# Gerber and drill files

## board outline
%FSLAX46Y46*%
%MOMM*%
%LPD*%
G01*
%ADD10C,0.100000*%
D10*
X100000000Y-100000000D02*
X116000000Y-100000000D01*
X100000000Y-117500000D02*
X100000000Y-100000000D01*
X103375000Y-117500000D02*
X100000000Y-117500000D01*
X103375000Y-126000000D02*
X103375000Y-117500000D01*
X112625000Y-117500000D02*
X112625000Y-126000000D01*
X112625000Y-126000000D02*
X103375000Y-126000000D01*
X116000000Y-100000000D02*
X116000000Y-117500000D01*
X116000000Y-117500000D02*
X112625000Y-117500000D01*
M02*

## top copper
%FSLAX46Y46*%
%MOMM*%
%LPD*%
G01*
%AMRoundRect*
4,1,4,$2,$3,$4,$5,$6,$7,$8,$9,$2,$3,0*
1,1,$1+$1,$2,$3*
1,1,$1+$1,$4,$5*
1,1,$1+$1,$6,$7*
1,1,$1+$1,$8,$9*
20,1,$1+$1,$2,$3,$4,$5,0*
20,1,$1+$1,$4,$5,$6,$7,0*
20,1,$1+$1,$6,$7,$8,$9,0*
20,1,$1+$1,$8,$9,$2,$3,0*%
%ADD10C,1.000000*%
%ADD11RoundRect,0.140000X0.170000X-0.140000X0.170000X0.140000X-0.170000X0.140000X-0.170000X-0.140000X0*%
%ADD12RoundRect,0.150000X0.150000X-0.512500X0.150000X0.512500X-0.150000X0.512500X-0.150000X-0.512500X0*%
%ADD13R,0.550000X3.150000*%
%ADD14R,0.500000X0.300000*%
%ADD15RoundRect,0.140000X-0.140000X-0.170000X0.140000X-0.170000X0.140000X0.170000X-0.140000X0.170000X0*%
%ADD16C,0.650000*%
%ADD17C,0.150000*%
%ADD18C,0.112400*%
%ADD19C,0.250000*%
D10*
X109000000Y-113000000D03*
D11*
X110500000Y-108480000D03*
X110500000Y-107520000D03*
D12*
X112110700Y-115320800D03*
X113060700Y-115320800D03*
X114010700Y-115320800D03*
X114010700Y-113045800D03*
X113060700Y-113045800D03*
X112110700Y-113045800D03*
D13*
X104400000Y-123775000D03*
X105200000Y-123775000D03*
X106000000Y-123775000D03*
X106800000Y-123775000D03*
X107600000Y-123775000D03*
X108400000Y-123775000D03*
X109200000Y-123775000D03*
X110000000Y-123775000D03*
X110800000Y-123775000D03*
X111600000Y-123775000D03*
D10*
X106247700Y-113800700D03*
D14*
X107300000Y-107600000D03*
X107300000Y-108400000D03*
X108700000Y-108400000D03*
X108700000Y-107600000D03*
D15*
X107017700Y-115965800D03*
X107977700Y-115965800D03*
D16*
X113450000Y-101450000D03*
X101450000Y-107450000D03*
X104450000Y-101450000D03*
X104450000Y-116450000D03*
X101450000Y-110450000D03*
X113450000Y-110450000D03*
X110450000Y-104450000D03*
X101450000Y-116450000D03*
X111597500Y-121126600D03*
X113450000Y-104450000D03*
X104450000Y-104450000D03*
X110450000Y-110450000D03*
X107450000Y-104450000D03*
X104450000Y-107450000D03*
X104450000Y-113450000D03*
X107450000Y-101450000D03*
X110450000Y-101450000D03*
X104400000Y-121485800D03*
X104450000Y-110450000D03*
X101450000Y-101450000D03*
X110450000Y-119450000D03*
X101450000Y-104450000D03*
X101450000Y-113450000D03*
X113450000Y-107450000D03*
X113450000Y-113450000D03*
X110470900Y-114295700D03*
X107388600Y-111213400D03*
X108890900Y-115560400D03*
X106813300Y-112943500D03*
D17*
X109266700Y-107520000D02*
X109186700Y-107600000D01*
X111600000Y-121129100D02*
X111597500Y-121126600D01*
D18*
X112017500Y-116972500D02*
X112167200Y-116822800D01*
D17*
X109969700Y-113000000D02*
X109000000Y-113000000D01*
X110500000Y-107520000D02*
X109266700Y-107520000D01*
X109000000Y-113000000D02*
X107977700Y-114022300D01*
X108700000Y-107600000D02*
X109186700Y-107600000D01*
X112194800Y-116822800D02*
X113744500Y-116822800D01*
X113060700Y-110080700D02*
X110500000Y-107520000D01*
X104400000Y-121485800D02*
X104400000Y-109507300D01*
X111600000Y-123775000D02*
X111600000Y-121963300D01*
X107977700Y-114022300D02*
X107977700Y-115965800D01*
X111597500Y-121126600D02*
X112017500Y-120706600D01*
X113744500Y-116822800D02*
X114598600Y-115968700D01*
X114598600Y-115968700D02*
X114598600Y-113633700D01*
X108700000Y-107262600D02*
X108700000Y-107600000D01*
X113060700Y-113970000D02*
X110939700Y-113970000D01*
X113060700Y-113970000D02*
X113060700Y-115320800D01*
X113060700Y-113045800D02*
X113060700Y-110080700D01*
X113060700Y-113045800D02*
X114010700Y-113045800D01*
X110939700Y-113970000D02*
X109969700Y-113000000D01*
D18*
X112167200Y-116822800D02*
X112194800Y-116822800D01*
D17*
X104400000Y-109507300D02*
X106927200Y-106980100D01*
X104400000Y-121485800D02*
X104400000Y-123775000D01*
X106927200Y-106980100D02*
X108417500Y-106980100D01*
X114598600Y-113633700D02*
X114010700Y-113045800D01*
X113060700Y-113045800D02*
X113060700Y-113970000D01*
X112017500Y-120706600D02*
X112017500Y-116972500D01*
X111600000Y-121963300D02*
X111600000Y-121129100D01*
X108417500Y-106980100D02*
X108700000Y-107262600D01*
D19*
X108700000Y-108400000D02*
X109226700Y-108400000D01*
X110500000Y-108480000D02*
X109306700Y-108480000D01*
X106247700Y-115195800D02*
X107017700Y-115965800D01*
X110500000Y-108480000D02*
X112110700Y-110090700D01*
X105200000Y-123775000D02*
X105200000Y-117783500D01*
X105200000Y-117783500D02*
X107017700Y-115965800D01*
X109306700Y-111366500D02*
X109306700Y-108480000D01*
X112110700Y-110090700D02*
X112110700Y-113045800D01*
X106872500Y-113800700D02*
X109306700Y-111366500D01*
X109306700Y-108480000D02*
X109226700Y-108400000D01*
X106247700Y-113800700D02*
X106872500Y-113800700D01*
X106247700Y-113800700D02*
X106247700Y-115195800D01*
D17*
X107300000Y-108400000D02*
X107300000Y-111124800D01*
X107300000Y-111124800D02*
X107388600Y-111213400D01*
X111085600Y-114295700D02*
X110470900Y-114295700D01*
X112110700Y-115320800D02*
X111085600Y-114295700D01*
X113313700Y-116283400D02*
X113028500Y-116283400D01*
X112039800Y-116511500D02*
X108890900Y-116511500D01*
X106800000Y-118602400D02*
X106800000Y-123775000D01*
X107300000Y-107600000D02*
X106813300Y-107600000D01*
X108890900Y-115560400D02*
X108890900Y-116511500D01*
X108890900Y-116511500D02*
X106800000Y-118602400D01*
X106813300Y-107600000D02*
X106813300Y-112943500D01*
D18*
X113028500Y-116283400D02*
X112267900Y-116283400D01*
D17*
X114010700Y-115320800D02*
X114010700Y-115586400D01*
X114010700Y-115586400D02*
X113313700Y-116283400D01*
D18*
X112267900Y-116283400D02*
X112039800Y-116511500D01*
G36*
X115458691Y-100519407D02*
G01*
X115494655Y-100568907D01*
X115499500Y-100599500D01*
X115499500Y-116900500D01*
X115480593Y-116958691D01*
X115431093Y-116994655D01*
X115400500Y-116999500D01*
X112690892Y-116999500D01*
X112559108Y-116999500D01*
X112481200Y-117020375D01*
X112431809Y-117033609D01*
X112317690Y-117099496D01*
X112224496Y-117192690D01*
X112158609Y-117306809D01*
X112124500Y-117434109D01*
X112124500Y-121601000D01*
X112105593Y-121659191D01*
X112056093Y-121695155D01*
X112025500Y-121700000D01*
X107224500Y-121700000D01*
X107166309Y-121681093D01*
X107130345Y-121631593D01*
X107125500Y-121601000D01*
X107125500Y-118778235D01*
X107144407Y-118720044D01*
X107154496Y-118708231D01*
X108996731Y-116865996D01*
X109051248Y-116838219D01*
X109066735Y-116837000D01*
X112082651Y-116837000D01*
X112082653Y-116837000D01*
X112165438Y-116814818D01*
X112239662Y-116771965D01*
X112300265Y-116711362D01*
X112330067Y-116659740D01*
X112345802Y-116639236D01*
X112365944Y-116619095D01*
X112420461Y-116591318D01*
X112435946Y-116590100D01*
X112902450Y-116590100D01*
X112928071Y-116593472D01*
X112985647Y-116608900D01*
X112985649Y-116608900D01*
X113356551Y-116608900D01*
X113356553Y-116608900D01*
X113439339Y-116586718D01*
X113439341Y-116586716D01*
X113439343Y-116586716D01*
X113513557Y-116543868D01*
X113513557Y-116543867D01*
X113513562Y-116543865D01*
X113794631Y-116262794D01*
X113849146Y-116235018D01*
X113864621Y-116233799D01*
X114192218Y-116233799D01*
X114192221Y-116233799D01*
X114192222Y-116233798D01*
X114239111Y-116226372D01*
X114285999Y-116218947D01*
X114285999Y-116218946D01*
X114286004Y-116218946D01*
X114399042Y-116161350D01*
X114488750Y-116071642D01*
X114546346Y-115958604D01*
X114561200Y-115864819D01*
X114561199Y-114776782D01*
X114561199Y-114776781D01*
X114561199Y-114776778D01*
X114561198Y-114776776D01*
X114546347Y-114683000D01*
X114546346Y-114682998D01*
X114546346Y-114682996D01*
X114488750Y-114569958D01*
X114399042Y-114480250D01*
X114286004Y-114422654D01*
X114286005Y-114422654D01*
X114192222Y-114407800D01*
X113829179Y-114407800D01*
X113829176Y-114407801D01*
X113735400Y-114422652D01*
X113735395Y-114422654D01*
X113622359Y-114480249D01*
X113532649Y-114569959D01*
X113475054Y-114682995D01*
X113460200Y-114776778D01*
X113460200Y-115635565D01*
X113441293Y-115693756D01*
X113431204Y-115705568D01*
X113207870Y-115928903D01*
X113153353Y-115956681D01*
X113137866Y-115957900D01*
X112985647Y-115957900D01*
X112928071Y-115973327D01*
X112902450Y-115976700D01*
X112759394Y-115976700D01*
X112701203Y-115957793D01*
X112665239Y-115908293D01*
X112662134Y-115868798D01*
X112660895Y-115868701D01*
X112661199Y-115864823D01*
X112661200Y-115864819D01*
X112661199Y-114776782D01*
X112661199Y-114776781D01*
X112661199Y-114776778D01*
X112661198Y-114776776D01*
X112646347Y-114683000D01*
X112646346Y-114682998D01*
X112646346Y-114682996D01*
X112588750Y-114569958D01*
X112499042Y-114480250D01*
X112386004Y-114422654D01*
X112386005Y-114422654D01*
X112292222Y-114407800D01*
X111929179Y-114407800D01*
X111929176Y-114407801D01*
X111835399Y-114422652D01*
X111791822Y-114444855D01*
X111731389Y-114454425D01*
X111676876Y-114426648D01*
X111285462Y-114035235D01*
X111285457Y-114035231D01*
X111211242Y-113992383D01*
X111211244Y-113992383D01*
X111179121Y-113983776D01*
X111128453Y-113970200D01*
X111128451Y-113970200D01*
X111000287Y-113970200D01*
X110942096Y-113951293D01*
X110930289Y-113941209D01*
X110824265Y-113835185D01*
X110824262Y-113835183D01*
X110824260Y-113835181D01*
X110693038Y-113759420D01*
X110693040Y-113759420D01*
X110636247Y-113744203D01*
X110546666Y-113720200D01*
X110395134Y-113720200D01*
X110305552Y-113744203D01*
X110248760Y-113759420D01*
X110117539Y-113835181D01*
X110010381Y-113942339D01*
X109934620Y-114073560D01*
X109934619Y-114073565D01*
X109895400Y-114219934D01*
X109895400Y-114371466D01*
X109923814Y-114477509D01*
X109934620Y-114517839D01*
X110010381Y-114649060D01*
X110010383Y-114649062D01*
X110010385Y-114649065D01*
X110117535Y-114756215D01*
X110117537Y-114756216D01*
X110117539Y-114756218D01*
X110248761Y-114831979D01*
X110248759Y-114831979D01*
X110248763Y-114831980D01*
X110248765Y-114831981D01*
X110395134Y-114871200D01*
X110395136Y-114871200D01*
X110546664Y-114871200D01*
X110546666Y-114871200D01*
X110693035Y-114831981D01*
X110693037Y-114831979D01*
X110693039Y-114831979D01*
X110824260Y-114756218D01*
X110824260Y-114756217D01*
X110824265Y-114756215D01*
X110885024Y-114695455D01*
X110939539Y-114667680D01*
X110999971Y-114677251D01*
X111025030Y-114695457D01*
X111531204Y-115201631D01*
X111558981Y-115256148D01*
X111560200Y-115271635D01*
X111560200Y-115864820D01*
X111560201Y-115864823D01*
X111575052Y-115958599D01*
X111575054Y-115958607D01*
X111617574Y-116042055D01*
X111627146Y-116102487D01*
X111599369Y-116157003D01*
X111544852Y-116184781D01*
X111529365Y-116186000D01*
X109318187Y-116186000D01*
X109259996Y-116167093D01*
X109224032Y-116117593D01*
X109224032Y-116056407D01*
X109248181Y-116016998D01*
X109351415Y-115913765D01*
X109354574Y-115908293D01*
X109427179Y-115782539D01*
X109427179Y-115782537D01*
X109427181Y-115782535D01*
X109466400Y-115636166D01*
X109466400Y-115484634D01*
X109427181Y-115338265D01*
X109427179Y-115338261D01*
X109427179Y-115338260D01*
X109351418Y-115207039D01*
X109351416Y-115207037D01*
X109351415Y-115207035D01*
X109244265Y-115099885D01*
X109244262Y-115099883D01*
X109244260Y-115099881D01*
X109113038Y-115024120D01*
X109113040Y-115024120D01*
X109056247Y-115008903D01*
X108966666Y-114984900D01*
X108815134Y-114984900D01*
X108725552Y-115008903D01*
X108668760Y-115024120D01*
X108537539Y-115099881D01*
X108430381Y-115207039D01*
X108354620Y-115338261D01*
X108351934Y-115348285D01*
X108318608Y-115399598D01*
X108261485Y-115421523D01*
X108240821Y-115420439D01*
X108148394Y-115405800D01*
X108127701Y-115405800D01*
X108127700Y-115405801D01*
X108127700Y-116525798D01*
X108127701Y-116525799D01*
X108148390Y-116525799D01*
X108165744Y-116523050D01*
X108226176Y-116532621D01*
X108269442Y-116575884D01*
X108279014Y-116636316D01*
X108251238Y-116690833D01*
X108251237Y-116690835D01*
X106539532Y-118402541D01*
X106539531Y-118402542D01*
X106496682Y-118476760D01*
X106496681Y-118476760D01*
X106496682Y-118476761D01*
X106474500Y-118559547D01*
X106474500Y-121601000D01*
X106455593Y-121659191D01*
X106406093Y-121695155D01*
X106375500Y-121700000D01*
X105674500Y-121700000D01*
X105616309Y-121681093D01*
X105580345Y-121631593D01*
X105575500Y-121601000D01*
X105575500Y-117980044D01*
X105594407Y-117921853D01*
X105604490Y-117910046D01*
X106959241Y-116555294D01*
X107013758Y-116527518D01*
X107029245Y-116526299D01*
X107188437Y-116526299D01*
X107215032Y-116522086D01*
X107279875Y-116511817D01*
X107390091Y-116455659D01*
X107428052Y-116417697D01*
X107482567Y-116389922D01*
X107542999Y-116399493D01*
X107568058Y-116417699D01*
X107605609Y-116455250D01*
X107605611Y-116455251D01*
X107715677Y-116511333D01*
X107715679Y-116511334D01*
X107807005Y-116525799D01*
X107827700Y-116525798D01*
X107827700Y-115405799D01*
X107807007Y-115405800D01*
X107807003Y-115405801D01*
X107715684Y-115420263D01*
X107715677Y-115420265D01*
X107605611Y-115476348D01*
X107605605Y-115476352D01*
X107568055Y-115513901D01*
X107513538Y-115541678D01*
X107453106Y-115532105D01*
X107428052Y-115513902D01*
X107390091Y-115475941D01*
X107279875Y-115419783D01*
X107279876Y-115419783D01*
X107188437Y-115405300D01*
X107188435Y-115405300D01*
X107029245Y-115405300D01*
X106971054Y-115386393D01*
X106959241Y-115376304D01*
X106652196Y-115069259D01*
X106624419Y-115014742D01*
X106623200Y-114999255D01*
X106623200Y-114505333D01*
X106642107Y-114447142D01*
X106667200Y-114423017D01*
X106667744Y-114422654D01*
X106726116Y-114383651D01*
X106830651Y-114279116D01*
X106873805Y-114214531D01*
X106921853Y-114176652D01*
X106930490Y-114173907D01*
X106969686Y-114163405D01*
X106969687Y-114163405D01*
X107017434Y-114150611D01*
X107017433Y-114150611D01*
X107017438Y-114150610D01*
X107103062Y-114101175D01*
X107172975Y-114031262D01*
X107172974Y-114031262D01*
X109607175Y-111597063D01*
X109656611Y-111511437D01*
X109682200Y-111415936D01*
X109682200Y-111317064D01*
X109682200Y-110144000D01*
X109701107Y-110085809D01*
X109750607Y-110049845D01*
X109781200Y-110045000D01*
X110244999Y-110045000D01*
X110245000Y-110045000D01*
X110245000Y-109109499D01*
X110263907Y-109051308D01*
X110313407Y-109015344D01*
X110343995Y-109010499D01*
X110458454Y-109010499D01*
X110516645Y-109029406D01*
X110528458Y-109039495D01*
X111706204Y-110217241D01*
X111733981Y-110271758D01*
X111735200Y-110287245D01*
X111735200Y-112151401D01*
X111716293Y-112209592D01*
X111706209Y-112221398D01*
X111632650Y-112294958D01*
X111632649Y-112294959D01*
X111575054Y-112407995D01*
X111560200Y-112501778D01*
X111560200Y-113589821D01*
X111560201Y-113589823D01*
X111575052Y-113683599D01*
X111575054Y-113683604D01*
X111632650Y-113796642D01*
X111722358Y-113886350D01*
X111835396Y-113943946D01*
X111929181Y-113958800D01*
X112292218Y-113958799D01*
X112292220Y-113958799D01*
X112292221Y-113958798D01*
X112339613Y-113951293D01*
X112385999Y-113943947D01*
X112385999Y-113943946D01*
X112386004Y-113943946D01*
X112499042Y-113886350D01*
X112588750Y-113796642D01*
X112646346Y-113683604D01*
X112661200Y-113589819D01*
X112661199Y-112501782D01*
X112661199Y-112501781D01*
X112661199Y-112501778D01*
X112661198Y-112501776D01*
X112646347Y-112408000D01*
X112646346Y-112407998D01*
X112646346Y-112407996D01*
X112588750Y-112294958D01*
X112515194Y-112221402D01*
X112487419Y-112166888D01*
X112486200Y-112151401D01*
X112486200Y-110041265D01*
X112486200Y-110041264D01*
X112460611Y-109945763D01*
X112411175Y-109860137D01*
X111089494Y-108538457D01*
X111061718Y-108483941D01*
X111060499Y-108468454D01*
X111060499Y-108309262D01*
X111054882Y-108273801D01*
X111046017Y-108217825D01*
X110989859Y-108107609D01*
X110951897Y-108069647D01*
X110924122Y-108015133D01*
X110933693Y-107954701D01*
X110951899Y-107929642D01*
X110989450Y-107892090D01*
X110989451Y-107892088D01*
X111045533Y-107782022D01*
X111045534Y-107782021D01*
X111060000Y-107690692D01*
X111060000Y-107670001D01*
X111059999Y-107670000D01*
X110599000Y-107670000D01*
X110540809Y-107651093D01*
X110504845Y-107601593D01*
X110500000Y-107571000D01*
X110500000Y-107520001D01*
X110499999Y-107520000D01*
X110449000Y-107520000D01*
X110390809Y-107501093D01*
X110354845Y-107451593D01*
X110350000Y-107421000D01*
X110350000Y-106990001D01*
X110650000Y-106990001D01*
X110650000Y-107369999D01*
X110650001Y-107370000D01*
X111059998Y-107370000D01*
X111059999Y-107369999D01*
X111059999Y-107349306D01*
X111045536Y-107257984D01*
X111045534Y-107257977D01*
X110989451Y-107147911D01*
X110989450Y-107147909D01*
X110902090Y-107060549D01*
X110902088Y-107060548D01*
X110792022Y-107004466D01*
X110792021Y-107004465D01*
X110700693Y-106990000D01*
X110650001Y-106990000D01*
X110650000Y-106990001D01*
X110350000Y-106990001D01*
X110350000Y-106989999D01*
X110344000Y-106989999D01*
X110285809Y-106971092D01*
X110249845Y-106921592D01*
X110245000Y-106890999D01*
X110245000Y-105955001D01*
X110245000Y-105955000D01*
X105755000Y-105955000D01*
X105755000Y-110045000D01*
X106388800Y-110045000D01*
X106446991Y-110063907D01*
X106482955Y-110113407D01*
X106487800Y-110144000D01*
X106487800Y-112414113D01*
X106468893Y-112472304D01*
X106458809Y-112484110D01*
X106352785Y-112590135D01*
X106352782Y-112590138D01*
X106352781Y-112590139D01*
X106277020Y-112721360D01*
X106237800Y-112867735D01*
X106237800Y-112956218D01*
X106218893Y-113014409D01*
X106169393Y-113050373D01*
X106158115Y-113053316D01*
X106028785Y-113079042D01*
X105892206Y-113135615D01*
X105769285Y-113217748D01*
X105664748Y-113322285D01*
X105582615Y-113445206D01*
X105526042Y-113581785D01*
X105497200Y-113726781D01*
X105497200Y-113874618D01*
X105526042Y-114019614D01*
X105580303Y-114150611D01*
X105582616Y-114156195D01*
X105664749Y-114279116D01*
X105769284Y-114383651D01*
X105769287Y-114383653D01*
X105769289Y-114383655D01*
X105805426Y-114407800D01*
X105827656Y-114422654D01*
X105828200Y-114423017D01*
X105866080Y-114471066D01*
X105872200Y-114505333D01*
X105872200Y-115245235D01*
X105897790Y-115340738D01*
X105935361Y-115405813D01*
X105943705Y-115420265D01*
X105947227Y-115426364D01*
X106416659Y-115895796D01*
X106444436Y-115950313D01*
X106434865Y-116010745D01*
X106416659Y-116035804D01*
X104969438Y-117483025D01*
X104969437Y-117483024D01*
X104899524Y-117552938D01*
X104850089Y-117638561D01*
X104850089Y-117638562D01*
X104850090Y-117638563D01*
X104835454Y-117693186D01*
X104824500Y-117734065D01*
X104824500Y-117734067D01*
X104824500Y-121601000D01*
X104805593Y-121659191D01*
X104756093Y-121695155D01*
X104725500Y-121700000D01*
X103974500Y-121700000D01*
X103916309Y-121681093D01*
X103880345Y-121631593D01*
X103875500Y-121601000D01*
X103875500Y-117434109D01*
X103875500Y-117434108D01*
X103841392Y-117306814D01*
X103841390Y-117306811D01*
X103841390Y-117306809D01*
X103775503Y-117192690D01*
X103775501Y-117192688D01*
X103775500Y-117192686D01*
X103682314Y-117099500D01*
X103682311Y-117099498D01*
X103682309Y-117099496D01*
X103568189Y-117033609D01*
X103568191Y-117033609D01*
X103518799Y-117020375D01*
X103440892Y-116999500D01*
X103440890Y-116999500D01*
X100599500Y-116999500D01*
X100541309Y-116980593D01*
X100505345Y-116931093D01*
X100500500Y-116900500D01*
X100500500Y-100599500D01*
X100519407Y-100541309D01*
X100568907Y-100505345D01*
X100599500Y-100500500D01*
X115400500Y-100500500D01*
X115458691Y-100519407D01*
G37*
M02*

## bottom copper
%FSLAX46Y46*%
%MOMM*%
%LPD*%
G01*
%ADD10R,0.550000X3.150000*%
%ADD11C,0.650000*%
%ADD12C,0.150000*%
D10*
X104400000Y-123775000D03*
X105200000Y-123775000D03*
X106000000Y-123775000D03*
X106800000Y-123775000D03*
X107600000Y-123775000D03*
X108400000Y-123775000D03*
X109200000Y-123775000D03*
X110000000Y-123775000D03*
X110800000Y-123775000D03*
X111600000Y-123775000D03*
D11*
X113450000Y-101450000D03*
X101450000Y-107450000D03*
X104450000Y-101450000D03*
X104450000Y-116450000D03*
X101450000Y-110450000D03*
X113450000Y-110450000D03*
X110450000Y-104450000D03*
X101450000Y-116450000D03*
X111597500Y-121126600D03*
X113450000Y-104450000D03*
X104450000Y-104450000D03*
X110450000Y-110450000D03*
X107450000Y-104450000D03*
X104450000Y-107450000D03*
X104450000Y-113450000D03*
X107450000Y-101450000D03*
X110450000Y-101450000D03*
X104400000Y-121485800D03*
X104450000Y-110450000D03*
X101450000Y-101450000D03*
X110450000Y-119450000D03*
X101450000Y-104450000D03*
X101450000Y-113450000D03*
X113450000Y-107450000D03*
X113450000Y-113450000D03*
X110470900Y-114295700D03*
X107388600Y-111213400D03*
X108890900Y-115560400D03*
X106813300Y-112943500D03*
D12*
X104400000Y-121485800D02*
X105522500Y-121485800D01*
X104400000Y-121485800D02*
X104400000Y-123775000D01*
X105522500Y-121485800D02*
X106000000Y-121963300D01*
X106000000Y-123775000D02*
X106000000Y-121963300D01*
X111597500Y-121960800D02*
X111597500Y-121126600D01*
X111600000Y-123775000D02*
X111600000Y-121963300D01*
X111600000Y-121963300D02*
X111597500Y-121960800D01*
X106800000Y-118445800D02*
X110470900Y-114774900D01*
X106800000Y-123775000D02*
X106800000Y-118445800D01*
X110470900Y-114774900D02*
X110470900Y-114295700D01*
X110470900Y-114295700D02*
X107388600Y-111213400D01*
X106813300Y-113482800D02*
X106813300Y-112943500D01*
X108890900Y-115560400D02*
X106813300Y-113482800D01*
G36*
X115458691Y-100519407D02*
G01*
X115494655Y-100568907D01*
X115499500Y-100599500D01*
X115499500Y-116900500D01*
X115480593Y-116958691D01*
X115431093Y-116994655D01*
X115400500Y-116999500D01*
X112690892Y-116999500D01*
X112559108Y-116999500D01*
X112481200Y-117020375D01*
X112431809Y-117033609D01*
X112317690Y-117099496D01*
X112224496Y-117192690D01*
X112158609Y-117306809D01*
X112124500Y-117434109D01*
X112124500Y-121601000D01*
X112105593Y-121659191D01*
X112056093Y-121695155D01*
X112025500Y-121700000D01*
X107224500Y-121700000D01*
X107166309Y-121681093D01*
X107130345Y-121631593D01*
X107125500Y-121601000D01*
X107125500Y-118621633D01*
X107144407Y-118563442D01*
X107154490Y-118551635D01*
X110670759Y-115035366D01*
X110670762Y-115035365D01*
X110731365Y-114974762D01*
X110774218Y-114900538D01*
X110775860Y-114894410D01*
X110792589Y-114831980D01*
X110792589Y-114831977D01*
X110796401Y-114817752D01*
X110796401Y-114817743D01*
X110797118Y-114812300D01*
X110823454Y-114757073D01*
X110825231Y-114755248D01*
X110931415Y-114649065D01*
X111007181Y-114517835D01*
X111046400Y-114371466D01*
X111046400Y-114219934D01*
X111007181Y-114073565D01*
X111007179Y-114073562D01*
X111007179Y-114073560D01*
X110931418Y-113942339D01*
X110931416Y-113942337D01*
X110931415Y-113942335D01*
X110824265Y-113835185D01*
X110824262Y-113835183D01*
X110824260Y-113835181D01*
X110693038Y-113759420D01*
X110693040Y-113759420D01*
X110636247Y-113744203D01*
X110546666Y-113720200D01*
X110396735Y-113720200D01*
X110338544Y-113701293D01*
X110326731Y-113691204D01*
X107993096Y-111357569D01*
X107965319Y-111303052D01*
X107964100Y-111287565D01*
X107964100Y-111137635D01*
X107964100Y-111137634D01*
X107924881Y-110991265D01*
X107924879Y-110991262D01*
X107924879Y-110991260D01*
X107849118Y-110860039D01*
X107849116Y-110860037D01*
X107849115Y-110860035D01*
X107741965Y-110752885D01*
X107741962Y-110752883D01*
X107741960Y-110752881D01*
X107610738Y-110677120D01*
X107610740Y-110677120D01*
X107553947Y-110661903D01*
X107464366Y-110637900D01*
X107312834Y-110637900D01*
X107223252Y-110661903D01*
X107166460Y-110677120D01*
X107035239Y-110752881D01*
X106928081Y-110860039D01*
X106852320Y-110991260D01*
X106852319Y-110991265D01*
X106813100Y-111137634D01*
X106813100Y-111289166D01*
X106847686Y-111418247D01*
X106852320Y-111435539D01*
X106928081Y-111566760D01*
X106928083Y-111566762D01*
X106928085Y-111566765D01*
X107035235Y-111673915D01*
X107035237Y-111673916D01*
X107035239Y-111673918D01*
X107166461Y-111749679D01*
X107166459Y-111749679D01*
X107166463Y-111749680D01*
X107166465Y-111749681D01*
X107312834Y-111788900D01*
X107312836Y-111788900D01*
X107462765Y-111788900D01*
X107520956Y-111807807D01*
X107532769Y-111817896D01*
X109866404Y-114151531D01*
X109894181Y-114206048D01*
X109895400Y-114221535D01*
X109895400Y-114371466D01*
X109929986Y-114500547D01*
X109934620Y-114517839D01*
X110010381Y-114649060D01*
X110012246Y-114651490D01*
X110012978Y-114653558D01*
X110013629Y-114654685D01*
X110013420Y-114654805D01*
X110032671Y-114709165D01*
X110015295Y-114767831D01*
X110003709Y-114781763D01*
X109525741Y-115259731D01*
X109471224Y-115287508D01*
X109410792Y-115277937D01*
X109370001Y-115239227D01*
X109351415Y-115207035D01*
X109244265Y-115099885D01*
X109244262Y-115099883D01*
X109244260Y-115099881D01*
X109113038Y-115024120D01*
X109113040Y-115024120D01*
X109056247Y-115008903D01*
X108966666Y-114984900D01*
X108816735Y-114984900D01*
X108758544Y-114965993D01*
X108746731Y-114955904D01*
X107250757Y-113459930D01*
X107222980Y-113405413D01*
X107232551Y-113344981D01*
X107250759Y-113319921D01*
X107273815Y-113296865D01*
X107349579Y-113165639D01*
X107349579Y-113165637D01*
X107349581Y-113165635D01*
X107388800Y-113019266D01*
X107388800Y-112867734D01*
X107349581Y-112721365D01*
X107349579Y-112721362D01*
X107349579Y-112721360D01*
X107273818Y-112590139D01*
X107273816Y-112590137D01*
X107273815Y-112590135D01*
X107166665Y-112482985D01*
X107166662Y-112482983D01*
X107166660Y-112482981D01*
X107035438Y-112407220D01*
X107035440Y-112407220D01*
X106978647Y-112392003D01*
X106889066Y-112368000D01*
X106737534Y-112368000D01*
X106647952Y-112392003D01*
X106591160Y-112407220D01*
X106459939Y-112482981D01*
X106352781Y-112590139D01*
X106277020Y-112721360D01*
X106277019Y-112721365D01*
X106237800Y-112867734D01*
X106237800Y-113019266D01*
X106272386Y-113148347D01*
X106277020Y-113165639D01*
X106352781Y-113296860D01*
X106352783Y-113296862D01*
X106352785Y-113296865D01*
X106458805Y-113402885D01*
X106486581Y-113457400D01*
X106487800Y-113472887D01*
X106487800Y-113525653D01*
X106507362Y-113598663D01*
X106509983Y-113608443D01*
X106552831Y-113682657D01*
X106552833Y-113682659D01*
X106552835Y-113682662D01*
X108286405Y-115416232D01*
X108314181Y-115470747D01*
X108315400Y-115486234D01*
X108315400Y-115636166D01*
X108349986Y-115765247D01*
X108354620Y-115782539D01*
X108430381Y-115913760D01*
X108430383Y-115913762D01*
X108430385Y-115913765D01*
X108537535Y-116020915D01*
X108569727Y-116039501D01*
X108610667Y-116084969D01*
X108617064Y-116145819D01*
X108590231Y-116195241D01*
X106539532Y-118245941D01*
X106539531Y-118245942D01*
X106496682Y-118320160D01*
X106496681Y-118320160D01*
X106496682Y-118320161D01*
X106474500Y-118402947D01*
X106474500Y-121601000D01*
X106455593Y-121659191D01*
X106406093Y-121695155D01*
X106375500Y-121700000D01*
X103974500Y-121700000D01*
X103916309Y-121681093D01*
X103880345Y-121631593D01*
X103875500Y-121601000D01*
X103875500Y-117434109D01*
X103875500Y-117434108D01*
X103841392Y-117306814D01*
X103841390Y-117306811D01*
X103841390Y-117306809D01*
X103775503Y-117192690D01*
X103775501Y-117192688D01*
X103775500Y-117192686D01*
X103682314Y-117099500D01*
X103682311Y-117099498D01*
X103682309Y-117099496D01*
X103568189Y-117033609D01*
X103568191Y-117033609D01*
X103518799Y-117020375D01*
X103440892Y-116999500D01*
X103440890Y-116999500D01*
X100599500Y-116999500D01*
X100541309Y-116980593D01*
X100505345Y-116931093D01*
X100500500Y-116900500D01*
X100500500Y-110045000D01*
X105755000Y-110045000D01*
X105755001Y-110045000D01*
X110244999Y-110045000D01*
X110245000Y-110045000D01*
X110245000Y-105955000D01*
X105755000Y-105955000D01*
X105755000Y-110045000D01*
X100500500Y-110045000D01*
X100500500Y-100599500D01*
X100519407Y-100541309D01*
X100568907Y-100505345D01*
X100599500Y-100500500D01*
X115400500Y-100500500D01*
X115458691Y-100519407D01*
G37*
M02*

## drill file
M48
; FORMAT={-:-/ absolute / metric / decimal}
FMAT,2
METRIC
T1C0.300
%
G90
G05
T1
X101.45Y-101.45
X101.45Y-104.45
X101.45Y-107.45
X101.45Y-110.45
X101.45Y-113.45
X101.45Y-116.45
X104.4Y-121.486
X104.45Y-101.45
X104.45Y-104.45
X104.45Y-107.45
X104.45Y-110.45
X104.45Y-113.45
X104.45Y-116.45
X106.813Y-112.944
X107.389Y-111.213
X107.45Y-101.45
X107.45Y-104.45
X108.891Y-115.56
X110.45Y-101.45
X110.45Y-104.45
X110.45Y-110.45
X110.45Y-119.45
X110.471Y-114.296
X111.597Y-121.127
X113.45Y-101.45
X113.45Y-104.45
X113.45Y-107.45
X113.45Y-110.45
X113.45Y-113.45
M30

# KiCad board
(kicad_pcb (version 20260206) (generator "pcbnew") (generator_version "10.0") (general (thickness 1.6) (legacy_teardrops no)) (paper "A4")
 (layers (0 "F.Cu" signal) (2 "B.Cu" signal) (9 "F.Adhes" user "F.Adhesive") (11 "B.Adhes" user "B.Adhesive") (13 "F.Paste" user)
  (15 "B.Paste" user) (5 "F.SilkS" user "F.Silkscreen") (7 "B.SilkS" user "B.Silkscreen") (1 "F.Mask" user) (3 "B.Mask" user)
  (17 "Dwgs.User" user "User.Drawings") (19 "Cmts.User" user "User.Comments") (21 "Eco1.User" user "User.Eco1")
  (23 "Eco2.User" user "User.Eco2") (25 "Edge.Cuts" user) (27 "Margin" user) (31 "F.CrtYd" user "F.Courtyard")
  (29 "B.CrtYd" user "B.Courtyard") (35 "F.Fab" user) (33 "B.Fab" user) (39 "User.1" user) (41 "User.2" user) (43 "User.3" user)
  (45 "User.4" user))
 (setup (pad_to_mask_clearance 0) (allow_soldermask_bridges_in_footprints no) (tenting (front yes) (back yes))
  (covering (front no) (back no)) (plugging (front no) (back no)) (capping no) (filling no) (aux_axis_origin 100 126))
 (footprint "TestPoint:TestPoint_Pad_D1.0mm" (layer "F.Cu") (at 109 113)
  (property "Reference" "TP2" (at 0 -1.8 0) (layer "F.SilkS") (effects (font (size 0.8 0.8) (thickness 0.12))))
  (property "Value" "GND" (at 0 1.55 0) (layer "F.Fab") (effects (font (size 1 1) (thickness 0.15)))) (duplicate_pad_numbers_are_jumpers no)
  (pad "1" smd circle (at 0 0) (size 1 1) (layers "F.Cu" "F.Mask") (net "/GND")))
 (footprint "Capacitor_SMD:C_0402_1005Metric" (layer "F.Cu") (at 110.5 108 90)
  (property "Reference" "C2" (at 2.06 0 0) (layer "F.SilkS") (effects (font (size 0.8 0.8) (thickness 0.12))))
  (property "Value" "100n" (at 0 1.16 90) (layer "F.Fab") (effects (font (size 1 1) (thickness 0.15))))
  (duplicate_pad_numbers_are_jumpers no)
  (pad "1" smd roundrect (at -0.48 0 90) (size 0.56 0.62) (layers "F.Cu" "F.Mask" "F.Paste") (roundrect_rratio 0.25) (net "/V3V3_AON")
   (zone_connect 1))
  (pad "2" smd roundrect (at 0.48 0 90) (size 0.56 0.62) (layers "F.Cu" "F.Mask" "F.Paste") (roundrect_rratio 0.25) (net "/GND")
   (zone_connect 1)))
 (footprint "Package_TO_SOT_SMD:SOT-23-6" (layer "F.Cu") (at 113.0607 114.1833 90)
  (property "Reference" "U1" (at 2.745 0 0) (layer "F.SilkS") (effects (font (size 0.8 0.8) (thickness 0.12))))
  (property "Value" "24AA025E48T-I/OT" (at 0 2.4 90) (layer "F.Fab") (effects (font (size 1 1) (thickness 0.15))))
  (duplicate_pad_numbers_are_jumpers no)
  (pad "1" smd roundrect (at -1.1375 -0.95 90) (size 1.325 0.6) (layers "F.Cu" "F.Mask" "F.Paste") (roundrect_rratio 0.25) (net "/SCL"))
  (pad "2" smd roundrect (at -1.1375 0 90) (size 1.325 0.6) (layers "F.Cu" "F.Mask" "F.Paste") (roundrect_rratio 0.25) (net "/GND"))
  (pad "3" smd roundrect (at -1.1375 0.95 90) (size 1.325 0.6) (layers "F.Cu" "F.Mask" "F.Paste") (roundrect_rratio 0.25) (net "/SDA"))
  (pad "4" smd roundrect (at 1.1375 0.95 90) (size 1.325 0.6) (layers "F.Cu" "F.Mask" "F.Paste") (roundrect_rratio 0.25) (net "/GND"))
  (pad "5" smd roundrect (at 1.1375 0 90) (size 1.325 0.6) (layers "F.Cu" "F.Mask" "F.Paste") (roundrect_rratio 0.25) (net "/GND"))
  (pad "6" smd roundrect (at 1.1375 -0.95 90) (size 1.325 0.6) (layers "F.Cu" "F.Mask" "F.Paste") (roundrect_rratio 0.25) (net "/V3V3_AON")))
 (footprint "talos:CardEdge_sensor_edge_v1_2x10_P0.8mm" (layer "F.Cu") (at 108 124.35)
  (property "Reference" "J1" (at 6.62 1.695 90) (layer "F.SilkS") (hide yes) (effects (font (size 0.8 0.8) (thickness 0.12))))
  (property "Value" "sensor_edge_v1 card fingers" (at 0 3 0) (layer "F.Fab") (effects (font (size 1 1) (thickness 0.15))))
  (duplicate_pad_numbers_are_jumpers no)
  (pad "1" smd rect (at -3.6 -0.575) (size 0.55 3.15) (layers "F.Cu" "F.Mask") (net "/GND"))
  (pad "2" smd rect (at -3.6 -0.575) (size 0.55 3.15) (layers "B.Cu" "B.Mask") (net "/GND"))
  (pad "3" smd rect (at -2.8 -0.575) (size 0.55 3.15) (layers "F.Cu" "F.Mask") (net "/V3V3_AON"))
  (pad "4" smd rect (at -2.8 -0.575) (size 0.55 3.15) (layers "B.Cu" "B.Mask") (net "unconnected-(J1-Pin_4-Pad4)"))
  (pad "5" smd rect (at -2 -0.575) (size 0.55 3.15) (layers "F.Cu" "F.Mask") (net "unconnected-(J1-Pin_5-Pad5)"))
  (pad "6" smd rect (at -2 -0.575) (size 0.55 3.15) (layers "B.Cu" "B.Mask") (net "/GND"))
  (pad "7" smd rect (at -1.2 -0.575) (size 0.55 3.15) (layers "F.Cu" "F.Mask") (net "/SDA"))
  (pad "8" smd rect (at -1.2 -0.575) (size 0.55 3.15) (layers "B.Cu" "B.Mask") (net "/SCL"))
  (pad "9" smd rect (at -0.4 -0.575) (size 0.55 3.15) (layers "F.Cu" "F.Mask") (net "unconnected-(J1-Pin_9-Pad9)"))
  (pad "10" smd rect (at -0.4 -0.575) (size 0.55 3.15) (layers "B.Cu" "B.Mask") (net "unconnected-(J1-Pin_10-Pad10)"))
  (pad "11" smd rect (at 0.4 -0.575) (size 0.55 3.15) (layers "F.Cu" "F.Mask") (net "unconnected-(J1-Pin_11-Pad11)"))
  (pad "12" smd rect (at 0.4 -0.575) (size 0.55 3.15) (layers "B.Cu" "B.Mask") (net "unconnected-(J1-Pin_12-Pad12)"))
  (pad "13" smd rect (at 1.2 -0.575) (size 0.55 3.15) (layers "F.Cu" "F.Mask") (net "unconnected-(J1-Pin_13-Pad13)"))
  (pad "14" smd rect (at 1.2 -0.575) (size 0.55 3.15) (layers "B.Cu" "B.Mask") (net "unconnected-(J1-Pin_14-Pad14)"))
  (pad "15" smd rect (at 2 -0.575) (size 0.55 3.15) (layers "F.Cu" "F.Mask") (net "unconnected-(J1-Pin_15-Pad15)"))
  (pad "16" smd rect (at 2 -0.575) (size 0.55 3.15) (layers "B.Cu" "B.Mask") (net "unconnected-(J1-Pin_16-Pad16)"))
  (pad "17" smd rect (at 2.8 -0.575) (size 0.55 3.15) (layers "F.Cu" "F.Mask") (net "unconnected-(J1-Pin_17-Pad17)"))
  (pad "18" smd rect (at 2.8 -0.575) (size 0.55 3.15) (layers "B.Cu" "B.Mask") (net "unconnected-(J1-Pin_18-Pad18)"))
  (pad "19" smd rect (at 3.6 -0.575) (size 0.55 3.15) (layers "F.Cu" "F.Mask") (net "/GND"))
  (pad "20" smd rect (at 3.6 -0.575) (size 0.55 3.15) (layers "B.Cu" "B.Mask") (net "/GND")))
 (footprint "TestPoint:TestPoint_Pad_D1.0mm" (layer "F.Cu") (at 106.2477 113.8007)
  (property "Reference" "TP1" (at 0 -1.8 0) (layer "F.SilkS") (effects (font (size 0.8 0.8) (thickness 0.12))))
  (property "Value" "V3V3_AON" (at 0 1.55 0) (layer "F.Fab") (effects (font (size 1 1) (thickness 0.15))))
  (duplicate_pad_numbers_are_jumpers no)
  (pad "1" smd circle (at 0 0) (size 1 1) (layers "F.Cu" "F.Mask") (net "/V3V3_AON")))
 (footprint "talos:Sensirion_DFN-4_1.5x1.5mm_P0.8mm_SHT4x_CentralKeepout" (layer "F.Cu") (at 108 108)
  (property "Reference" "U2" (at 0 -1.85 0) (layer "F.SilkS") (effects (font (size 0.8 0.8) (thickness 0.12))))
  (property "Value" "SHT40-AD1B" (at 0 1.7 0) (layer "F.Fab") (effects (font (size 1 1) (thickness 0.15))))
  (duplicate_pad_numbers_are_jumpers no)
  (pad "1" smd rect (at -0.7 -0.4) (size 0.5 0.3) (layers "F.Cu" "F.Mask" "F.Paste") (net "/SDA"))
  (pad "2" smd rect (at -0.7 0.4) (size 0.5 0.3) (layers "F.Cu" "F.Mask" "F.Paste") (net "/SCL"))
  (pad "3" smd rect (at 0.7 0.4) (size 0.5 0.3) (layers "F.Cu" "F.Mask" "F.Paste") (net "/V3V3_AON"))
  (pad "4" smd rect (at 0.7 -0.4) (size 0.5 0.3) (layers "F.Cu" "F.Mask" "F.Paste") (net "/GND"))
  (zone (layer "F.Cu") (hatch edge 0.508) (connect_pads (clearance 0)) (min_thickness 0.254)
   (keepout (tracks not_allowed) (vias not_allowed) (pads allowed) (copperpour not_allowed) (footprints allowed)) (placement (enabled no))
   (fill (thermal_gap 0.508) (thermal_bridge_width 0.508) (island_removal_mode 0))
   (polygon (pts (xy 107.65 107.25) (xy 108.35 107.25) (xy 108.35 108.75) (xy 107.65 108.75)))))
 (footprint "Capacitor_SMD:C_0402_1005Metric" (layer "F.Cu") (at 107.4977 115.9658)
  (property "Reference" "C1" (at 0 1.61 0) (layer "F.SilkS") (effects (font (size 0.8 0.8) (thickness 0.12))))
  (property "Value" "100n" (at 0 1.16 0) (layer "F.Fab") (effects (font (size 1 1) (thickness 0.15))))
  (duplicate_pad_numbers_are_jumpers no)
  (pad "1" smd roundrect (at -0.48 0) (size 0.56 0.62) (layers "F.Cu" "F.Mask" "F.Paste") (roundrect_rratio 0.25) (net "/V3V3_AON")
   (zone_connect 1))
  (pad "2" smd roundrect (at 0.48 0) (size 0.56 0.62) (layers "F.Cu" "F.Mask" "F.Paste") (roundrect_rratio 0.25) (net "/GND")
   (zone_connect 1)))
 (gr_line (start 100 100) (end 116 100) (stroke (width 0.1) (type default)) (layer "Edge.Cuts"))
 (gr_line (start 100 117.5) (end 100 100) (stroke (width 0.1) (type default)) (layer "Edge.Cuts"))
 (gr_line (start 103.375 117.5) (end 100 117.5) (stroke (width 0.1) (type default)) (layer "Edge.Cuts"))
 (gr_line (start 103.375 126) (end 103.375 117.5) (stroke (width 0.1) (type default)) (layer "Edge.Cuts"))
 (gr_line (start 112.625 117.5) (end 112.625 126) (stroke (width 0.1) (type default)) (layer "Edge.Cuts"))
 (gr_line (start 112.625 126) (end 103.375 126) (stroke (width 0.1) (type default)) (layer "Edge.Cuts"))
 (gr_line (start 116 100) (end 116 117.5) (stroke (width 0.1) (type default)) (layer "Edge.Cuts"))
 (gr_line (start 116 117.5) (end 112.625 117.5) (stroke (width 0.1) (type default)) (layer "Edge.Cuts"))
 (segment (start 109.2667 107.52) (end 109.1867 107.6) (width 0.15) (layer "F.Cu") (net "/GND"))
 (segment (start 111.6 121.1291) (end 111.5975 121.1266) (width 0.15) (layer "F.Cu") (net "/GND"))
 (segment (start 112.0175 116.9725) (end 112.1672 116.8228) (width 0.1124) (layer "F.Cu") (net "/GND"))
 (segment (start 109.9697 113) (end 109 113) (width 0.15) (layer "F.Cu") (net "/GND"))
 (segment (start 110.5 107.52) (end 109.2667 107.52) (width 0.15) (layer "F.Cu") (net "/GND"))
 (segment (start 109 113) (end 107.9777 114.0223) (width 0.15) (layer "F.Cu") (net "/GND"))
 (segment (start 108.7 107.6) (end 109.1867 107.6) (width 0.15) (layer "F.Cu") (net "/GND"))
 (segment (start 112.1948 116.8228) (end 113.7445 116.8228) (width 0.15) (layer "F.Cu") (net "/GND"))
 (segment (start 113.0607 110.0807) (end 110.5 107.52) (width 0.15) (layer "F.Cu") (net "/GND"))
 (segment (start 104.4 121.4858) (end 104.4 109.5073) (width 0.15) (layer "F.Cu") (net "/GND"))
 (segment (start 111.6 123.775) (end 111.6 121.9633) (width 0.15) (layer "F.Cu") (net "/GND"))
 (segment (start 107.9777 114.0223) (end 107.9777 115.9658) (width 0.15) (layer "F.Cu") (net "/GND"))
 (segment (start 111.5975 121.1266) (end 112.0175 120.7066) (width 0.15) (layer "F.Cu") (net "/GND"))
 (segment (start 113.7445 116.8228) (end 114.5986 115.9687) (width 0.15) (layer "F.Cu") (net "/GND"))
 (segment (start 114.5986 115.9687) (end 114.5986 113.6337) (width 0.15) (layer "F.Cu") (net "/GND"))
 (segment (start 108.7 107.2626) (end 108.7 107.6) (width 0.15) (layer "F.Cu") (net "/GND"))
 (segment (start 113.0607 113.97) (end 110.9397 113.97) (width 0.15) (layer "F.Cu") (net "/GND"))
 (segment (start 113.0607 113.97) (end 113.0607 115.3208) (width 0.15) (layer "F.Cu") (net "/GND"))
 (segment (start 113.0607 113.0458) (end 113.0607 110.0807) (width 0.15) (layer "F.Cu") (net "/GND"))
 (segment (start 113.0607 113.0458) (end 114.0107 113.0458) (width 0.15) (layer "F.Cu") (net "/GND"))
 (segment (start 110.9397 113.97) (end 109.9697 113) (width 0.15) (layer "F.Cu") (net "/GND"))
 (segment (start 112.1672 116.8228) (end 112.1948 116.8228) (width 0.1124) (layer "F.Cu") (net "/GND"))
 (segment (start 104.4 109.5073) (end 106.9272 106.9801) (width 0.15) (layer "F.Cu") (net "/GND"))
 (segment (start 104.4 121.4858) (end 104.4 123.775) (width 0.15) (layer "F.Cu") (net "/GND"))
 (segment (start 106.9272 106.9801) (end 108.4175 106.9801) (width 0.15) (layer "F.Cu") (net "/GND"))
 (segment (start 114.5986 113.6337) (end 114.0107 113.0458) (width 0.15) (layer "F.Cu") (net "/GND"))
 (segment (start 113.0607 113.0458) (end 113.0607 113.97) (width 0.15) (layer "F.Cu") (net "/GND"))
 (segment (start 112.0175 120.7066) (end 112.0175 116.9725) (width 0.15) (layer "F.Cu") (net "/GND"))
 (segment (start 111.6 121.9633) (end 111.6 121.1291) (width 0.15) (layer "F.Cu") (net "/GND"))
 (segment (start 108.4175 106.9801) (end 108.7 107.2626) (width 0.15) (layer "F.Cu") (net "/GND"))
 (via (at 113.45 101.45) (size 0.65) (drill 0.3) (layers "F.Cu" "B.Cu") (locked yes) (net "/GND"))
 (via (at 101.45 107.45) (size 0.65) (drill 0.3) (layers "F.Cu" "B.Cu") (locked yes) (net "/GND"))
 (via (at 104.45 101.45) (size 0.65) (drill 0.3) (layers "F.Cu" "B.Cu") (locked yes) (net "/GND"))
 (via (at 104.45 116.45) (size 0.65) (drill 0.3) (layers "F.Cu" "B.Cu") (locked yes) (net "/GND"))
 (via (at 101.45 110.45) (size 0.65) (drill 0.3) (layers "F.Cu" "B.Cu") (locked yes) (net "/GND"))
 (via (at 113.45 110.45) (size 0.65) (drill 0.3) (layers "F.Cu" "B.Cu") (locked yes) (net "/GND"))
 (via (at 110.45 104.45) (size 0.65) (drill 0.3) (layers "F.Cu" "B.Cu") (locked yes) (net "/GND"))
 (via (at 101.45 116.45) (size 0.65) (drill 0.3) (layers "F.Cu" "B.Cu") (locked yes) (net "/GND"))
 (via (at 111.5975 121.1266) (size 0.65) (drill 0.3) (layers "F.Cu" "B.Cu") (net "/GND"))
 (via (at 113.45 104.45) (size 0.65) (drill 0.3) (layers "F.Cu" "B.Cu") (locked yes) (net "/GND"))
 (via (at 104.45 104.45) (size 0.65) (drill 0.3) (layers "F.Cu" "B.Cu") (locked yes) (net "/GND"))
 (via (at 110.45 110.45) (size 0.65) (drill 0.3) (layers "F.Cu" "B.Cu") (locked yes) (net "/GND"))
 (via (at 107.45 104.45) (size 0.65) (drill 0.3) (layers "F.Cu" "B.Cu") (locked yes) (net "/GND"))
 (via (at 104.45 107.45) (size 0.65) (drill 0.3) (layers "F.Cu" "B.Cu") (locked yes) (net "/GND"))
 (via (at 104.45 113.45) (size 0.65) (drill 0.3) (layers "F.Cu" "B.Cu") (locked yes) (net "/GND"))
 (via (at 107.45 101.45) (size 0.65) (drill 0.3) (layers "F.Cu" "B.Cu") (locked yes) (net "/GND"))
 (via (at 110.45 101.45) (size 0.65) (drill 0.3) (layers "F.Cu" "B.Cu") (locked yes) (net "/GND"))
 (via (at 104.4 121.4858) (size 0.65) (drill 0.3) (layers "F.Cu" "B.Cu") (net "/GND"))
 (via (at 104.45 110.45) (size 0.65) (drill 0.3) (layers "F.Cu" "B.Cu") (locked yes) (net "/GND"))
 (via (at 101.45 101.45) (size 0.65) (drill 0.3) (layers "F.Cu" "B.Cu") (locked yes) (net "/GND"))
 (via (at 110.45 119.45) (size 0.65) (drill 0.3) (layers "F.Cu" "B.Cu") (locked yes) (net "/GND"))
 (via (at 101.45 104.45) (size 0.65) (drill 0.3) (layers "F.Cu" "B.Cu") (locked yes) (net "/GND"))
 (via (at 101.45 113.45) (size 0.65) (drill 0.3) (layers "F.Cu" "B.Cu") (locked yes) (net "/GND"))
 (via (at 113.45 107.45) (size 0.65) (drill 0.3) (layers "F.Cu" "B.Cu") (locked yes) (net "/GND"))
 (via (at 113.45 113.45) (size 0.65) (drill 0.3) (layers "F.Cu" "B.Cu") (locked yes) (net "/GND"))
 (segment (start 104.4 121.4858) (end 105.5225 121.4858) (width 0.15) (layer "B.Cu") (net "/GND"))
 (segment (start 104.4 121.4858) (end 104.4 123.775) (width 0.15) (layer "B.Cu") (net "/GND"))
 (segment (start 105.5225 121.4858) (end 106 121.9633) (width 0.15) (layer "B.Cu") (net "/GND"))
 (segment (start 106 123.775) (end 106 121.9633) (width 0.15) (layer "B.Cu") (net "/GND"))
 (segment (start 111.5975 121.9608) (end 111.5975 121.1266) (width 0.15) (layer "B.Cu") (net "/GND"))
 (segment (start 111.6 123.775) (end 111.6 121.9633) (width 0.15) (layer "B.Cu") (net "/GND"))
 (segment (start 111.6 121.9633) (end 111.5975 121.9608) (width 0.15) (layer "B.Cu") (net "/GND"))
 (segment (start 108.7 108.4) (end 109.2267 108.4) (width 0.25) (layer "F.Cu") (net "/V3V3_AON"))
 (segment (start 110.5 108.48) (end 109.3067 108.48) (width 0.25) (layer "F.Cu") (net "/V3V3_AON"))
 (segment (start 106.2477 115.1958) (end 107.0177 115.9658) (width 0.25) (layer "F.Cu") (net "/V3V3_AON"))
 (segment (start 110.5 108.48) (end 112.1107 110.0907) (width 0.25) (layer "F.Cu") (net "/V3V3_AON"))
 (segment (start 105.2 123.775) (end 105.2 117.7835) (width 0.25) (layer "F.Cu") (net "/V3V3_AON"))
 (segment (start 105.2 117.7835) (end 107.0177 115.9658) (width 0.25) (layer "F.Cu") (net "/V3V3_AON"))
 (segment (start 109.3067 111.3665) (end 109.3067 108.48) (width 0.25) (layer "F.Cu") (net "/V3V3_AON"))
 (segment (start 112.1107 110.0907) (end 112.1107 113.0458) (width 0.25) (layer "F.Cu") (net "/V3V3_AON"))
 (segment (start 106.8725 113.8007) (end 109.3067 111.3665) (width 0.25) (layer "F.Cu") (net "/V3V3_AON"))
 (segment (start 109.3067 108.48) (end 109.2267 108.4) (width 0.25) (layer "F.Cu") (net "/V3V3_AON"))
 (segment (start 106.2477 113.8007) (end 106.8725 113.8007) (width 0.25) (layer "F.Cu") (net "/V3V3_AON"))
 (segment (start 106.2477 113.8007) (end 106.2477 115.1958) (width 0.25) (layer "F.Cu") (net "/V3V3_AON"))
 (segment (start 107.3 108.4) (end 107.3 111.1248) (width 0.15) (layer "F.Cu") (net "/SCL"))
 (segment (start 107.3 111.1248) (end 107.3886 111.2134) (width 0.15) (layer "F.Cu") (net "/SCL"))
 (segment (start 111.0856 114.2957) (end 110.4709 114.2957) (width 0.15) (layer "F.Cu") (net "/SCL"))
 (segment (start 112.1107 115.3208) (end 111.0856 114.2957) (width 0.15) (layer "F.Cu") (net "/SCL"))
 (via (at 110.4709 114.2957) (size 0.65) (drill 0.3) (layers "F.Cu" "B.Cu") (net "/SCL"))
 (via (at 107.3886 111.2134) (size 0.65) (drill 0.3) (layers "F.Cu" "B.Cu") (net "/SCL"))
 (segment (start 106.8 118.4458) (end 110.4709 114.7749) (width 0.15) (layer "B.Cu") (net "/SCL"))
 (segment (start 106.8 123.775) (end 106.8 118.4458) (width 0.15) (layer "B.Cu") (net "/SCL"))
 (segment (start 110.4709 114.7749) (end 110.4709 114.2957) (width 0.15) (layer "B.Cu") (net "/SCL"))
 (segment (start 110.4709 114.2957) (end 107.3886 111.2134) (width 0.15) (layer "B.Cu") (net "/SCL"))
 (segment (start 113.3137 116.2834) (end 113.0285 116.2834) (width 0.15) (layer "F.Cu") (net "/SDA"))
 (segment (start 112.0398 116.5115) (end 108.8909 116.5115) (width 0.15) (layer "F.Cu") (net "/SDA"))
 (segment (start 106.8 118.6024) (end 106.8 123.775) (width 0.15) (layer "F.Cu") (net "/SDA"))
 (segment (start 107.3 107.6) (end 106.8133 107.6) (width 0.15) (layer "F.Cu") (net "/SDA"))
 (segment (start 108.8909 115.5604) (end 108.8909 116.5115) (width 0.15) (layer "F.Cu") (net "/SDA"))
 (segment (start 108.8909 116.5115) (end 106.8 118.6024) (width 0.15) (layer "F.Cu") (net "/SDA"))
 (segment (start 106.8133 107.6) (end 106.8133 112.9435) (width 0.15) (layer "F.Cu") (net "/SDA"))
 (segment (start 113.0285 116.2834) (end 112.2679 116.2834) (width 0.1124) (layer "F.Cu") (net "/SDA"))
 (segment (start 114.0107 115.3208) (end 114.0107 115.5864) (width 0.15) (layer "F.Cu") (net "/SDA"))
 (segment (start 114.0107 115.5864) (end 113.3137 116.2834) (width 0.15) (layer "F.Cu") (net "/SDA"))
 (segment (start 112.2679 116.2834) (end 112.0398 116.5115) (width 0.1124) (layer "F.Cu") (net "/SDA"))
 (via (at 108.8909 115.5604) (size 0.65) (drill 0.3) (layers "F.Cu" "B.Cu") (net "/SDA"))
 (via (at 106.8133 112.9435) (size 0.65) (drill 0.3) (layers "F.Cu" "B.Cu") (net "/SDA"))
 (segment (start 106.8133 113.4828) (end 106.8133 112.9435) (width 0.15) (layer "B.Cu") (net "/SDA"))
 (segment (start 108.8909 115.5604) (end 106.8133 113.4828) (width 0.15) (layer "B.Cu") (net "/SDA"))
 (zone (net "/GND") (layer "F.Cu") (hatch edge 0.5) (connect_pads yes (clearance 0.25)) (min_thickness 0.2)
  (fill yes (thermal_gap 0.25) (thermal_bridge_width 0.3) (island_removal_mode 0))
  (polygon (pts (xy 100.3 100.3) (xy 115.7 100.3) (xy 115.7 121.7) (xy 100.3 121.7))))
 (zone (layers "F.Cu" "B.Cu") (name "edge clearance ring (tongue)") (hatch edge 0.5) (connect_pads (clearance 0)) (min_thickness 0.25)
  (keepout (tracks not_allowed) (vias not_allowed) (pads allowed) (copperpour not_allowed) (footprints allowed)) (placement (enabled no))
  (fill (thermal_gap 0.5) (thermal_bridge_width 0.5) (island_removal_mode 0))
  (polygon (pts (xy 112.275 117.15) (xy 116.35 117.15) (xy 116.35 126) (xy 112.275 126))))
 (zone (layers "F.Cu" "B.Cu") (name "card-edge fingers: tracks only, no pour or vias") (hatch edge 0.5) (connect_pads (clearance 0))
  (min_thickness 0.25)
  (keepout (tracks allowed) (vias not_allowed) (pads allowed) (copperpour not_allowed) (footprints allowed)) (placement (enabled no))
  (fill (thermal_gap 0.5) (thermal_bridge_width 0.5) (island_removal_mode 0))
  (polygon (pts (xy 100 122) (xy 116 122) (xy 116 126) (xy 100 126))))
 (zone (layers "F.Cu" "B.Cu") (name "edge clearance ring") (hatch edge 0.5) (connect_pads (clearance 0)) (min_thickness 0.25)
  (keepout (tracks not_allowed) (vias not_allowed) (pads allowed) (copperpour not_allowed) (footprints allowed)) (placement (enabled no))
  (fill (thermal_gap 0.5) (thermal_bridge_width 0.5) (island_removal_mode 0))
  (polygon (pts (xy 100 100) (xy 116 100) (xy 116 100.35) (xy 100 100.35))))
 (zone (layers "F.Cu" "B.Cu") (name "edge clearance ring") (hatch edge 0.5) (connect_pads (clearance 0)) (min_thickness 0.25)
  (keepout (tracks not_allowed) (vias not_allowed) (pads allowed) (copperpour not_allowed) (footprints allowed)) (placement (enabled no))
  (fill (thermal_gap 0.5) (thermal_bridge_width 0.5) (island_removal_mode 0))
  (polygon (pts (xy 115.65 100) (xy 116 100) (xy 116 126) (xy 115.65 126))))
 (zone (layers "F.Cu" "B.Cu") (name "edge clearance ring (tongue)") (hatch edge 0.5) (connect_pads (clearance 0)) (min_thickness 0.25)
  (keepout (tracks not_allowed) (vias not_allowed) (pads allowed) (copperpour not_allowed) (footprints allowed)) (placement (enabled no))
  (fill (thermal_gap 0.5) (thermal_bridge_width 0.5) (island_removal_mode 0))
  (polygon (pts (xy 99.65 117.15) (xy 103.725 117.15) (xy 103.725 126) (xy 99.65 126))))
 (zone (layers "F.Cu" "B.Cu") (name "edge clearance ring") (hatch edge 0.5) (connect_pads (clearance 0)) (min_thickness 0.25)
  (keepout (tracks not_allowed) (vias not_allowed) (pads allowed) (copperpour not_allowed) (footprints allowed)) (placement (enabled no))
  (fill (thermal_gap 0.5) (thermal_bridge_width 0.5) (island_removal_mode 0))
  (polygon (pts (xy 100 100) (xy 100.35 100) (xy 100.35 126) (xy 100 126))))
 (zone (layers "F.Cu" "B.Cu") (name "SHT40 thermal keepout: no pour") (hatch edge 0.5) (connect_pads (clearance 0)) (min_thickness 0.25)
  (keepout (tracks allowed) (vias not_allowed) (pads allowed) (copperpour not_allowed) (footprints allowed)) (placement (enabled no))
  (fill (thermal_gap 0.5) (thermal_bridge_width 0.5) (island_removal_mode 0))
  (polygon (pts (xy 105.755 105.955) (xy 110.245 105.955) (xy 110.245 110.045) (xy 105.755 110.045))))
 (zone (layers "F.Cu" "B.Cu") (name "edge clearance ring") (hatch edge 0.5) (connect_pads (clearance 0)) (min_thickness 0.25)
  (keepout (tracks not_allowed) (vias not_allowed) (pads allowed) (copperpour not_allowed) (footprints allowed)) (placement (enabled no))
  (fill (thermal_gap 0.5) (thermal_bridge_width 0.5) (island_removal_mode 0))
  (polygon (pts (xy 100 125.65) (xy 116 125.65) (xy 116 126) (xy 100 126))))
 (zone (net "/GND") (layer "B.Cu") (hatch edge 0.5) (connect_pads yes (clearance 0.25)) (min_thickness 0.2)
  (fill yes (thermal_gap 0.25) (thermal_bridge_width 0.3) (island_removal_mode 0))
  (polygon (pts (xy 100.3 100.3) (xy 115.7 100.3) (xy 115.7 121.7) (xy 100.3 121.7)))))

